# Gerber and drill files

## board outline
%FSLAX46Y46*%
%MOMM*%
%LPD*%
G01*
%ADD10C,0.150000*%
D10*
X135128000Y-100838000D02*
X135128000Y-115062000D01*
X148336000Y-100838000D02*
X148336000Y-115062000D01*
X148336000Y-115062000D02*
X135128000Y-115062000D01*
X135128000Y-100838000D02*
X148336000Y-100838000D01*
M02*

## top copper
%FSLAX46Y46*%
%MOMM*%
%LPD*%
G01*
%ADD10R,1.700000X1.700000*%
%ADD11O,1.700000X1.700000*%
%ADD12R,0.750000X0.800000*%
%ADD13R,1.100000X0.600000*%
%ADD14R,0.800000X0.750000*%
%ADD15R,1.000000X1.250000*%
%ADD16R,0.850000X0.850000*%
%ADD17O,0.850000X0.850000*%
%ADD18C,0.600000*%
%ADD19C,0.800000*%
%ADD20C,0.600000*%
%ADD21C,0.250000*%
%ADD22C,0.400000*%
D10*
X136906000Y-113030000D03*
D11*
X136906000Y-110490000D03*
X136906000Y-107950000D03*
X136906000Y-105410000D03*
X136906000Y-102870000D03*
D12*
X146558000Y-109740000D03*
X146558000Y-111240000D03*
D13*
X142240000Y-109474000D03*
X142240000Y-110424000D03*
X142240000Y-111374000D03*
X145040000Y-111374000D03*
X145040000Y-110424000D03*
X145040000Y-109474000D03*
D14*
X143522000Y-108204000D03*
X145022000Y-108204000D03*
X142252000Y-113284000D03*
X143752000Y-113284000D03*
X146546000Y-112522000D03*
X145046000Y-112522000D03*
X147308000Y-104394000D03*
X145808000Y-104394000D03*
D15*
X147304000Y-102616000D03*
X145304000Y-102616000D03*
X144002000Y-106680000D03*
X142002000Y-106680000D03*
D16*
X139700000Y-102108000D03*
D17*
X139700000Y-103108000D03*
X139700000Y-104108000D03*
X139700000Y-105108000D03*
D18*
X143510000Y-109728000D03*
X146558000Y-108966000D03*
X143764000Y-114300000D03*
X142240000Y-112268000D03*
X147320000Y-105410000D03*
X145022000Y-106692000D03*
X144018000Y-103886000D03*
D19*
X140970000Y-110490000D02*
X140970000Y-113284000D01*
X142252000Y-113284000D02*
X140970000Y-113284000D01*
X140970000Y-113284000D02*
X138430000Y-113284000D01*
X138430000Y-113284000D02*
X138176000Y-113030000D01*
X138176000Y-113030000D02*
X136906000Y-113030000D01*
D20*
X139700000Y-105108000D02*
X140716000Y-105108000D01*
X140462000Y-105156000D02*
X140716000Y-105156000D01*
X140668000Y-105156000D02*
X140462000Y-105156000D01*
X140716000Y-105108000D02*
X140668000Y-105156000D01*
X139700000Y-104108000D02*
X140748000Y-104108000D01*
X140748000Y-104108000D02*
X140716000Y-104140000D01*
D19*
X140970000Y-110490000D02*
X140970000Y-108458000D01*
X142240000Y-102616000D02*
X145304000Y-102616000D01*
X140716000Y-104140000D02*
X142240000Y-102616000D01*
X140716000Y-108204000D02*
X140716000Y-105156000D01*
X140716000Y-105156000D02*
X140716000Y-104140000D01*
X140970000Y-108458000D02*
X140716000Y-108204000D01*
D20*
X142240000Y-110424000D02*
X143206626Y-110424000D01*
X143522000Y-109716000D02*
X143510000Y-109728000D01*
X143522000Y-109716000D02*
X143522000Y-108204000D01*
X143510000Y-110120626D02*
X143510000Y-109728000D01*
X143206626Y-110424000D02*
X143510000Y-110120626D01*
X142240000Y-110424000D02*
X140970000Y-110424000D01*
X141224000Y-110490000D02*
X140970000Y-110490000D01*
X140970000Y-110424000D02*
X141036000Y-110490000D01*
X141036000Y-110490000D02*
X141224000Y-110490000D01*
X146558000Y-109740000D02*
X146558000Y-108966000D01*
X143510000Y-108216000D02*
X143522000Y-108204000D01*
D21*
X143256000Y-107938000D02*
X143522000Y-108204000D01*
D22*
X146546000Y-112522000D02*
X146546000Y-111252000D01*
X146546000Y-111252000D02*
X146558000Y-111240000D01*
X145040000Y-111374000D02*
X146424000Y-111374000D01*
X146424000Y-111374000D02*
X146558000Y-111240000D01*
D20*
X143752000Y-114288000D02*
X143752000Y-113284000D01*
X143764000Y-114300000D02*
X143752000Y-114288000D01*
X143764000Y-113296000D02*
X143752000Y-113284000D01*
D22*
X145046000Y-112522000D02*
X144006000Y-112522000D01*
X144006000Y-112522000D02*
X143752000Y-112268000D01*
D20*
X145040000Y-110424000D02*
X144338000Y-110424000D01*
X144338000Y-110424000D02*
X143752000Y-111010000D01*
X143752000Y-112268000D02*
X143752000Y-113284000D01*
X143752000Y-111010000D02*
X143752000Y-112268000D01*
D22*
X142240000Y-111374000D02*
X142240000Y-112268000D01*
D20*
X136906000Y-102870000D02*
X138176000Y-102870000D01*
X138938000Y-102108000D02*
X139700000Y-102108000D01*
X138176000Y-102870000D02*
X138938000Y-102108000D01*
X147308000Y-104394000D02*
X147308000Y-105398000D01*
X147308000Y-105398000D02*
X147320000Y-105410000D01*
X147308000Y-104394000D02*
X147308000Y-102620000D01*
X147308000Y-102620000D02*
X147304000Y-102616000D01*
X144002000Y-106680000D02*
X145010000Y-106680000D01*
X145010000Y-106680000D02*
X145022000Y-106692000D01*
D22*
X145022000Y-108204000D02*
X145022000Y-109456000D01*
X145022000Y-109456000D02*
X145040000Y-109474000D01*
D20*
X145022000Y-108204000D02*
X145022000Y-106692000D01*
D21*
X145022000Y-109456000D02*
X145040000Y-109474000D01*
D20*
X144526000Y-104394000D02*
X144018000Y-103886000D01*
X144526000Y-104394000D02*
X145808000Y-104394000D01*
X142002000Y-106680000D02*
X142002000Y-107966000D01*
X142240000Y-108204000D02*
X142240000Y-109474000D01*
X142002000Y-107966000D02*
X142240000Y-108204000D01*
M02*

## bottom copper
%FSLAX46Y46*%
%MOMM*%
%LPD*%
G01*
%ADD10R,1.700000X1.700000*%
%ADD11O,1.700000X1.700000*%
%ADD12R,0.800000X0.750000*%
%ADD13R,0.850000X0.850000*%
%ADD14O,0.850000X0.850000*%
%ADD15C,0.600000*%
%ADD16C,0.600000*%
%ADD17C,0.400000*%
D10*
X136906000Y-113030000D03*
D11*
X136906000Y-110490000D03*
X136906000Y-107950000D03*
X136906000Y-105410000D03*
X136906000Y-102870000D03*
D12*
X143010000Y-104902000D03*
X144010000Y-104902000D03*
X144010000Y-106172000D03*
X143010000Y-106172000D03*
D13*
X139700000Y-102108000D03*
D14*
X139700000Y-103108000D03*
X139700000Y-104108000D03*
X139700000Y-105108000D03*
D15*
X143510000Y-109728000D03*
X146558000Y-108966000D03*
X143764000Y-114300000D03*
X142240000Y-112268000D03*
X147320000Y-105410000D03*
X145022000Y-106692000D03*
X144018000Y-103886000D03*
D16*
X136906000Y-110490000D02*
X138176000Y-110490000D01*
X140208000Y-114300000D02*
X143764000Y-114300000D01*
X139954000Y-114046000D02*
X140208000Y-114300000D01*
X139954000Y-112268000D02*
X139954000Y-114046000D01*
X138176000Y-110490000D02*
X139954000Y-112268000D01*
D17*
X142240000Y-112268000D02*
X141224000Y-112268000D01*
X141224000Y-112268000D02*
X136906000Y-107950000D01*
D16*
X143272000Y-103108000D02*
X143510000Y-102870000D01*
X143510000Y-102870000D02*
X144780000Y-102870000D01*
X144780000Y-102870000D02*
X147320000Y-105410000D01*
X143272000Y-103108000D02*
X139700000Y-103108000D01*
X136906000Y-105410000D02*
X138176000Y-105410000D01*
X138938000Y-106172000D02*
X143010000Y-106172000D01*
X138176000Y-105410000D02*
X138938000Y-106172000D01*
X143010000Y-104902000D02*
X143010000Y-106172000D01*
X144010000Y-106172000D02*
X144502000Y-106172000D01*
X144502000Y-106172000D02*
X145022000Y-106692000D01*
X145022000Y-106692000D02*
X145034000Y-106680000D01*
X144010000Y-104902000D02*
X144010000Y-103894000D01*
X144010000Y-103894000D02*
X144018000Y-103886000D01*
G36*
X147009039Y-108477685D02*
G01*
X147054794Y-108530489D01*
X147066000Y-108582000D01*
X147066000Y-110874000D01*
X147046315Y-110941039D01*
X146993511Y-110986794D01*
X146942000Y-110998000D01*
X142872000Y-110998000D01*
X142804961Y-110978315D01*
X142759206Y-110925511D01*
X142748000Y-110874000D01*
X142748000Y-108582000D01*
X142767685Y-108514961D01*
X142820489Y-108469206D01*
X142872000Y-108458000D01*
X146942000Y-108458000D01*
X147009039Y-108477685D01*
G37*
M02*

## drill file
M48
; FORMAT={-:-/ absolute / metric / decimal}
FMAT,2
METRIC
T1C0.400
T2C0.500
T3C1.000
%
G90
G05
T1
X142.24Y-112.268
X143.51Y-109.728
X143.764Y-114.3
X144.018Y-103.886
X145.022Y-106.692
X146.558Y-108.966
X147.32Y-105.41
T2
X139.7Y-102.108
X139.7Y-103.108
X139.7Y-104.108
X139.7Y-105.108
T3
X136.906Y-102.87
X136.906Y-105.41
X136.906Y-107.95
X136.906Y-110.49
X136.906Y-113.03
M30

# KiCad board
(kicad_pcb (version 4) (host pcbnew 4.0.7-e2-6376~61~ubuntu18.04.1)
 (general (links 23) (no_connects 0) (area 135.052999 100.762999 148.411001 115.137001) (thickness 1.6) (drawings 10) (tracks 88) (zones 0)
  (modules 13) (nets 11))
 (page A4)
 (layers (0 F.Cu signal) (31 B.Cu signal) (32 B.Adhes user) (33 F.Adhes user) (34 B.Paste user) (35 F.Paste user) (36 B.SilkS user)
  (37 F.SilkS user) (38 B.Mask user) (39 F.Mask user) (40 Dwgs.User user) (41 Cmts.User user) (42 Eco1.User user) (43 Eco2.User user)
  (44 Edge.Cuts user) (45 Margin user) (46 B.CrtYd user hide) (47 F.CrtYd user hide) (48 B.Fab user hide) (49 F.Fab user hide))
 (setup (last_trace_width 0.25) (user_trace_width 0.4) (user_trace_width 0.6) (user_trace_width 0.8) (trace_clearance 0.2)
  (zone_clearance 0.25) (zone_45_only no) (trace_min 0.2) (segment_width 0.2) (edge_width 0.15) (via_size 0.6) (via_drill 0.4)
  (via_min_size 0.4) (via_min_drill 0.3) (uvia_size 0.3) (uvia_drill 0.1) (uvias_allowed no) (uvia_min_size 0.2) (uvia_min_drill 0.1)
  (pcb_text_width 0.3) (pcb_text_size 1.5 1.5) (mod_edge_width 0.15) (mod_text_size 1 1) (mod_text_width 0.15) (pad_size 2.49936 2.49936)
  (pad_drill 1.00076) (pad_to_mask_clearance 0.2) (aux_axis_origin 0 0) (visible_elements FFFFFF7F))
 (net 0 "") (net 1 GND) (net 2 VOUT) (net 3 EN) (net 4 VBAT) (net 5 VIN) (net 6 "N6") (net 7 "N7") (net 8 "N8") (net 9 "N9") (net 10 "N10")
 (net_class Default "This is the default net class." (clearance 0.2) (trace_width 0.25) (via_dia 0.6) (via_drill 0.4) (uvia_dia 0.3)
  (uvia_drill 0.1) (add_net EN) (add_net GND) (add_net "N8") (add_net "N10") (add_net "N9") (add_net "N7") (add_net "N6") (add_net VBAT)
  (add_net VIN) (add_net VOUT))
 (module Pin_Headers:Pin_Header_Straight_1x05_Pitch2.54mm (layer F.Cu) (at 136.906 113.03 180)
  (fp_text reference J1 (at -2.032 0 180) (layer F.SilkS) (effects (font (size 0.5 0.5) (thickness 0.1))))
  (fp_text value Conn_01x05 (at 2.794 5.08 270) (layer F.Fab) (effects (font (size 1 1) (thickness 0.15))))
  (pad 1 thru_hole rect (at 0 0 180) (size 1.7 1.7) (drill 1) (layers *.Cu *.Mask) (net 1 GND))
  (pad 2 thru_hole oval (at 0 2.54 180) (size 1.7 1.7) (drill 1) (layers *.Cu *.Mask) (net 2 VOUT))
  (pad 3 thru_hole oval (at 0 5.08 180) (size 1.7 1.7) (drill 1) (layers *.Cu *.Mask) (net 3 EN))
  (pad 4 thru_hole oval (at 0 7.62 180) (size 1.7 1.7) (drill 1) (layers *.Cu *.Mask) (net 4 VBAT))
  (pad 5 thru_hole oval (at 0 10.16 180) (size 1.7 1.7) (drill 1) (layers *.Cu *.Mask) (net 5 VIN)))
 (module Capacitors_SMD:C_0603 (layer F.Cu) (at 146.558 110.49 90)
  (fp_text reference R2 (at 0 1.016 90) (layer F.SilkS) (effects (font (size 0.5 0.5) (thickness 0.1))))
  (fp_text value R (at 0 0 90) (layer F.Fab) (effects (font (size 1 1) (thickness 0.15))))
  (pad 2 smd rect (at 0.75 0 90) (size 0.8 0.75) (layers F.Cu F.Paste F.Mask) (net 1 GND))
  (pad 1 smd rect (at -0.75 0 90) (size 0.8 0.75) (layers F.Cu F.Paste F.Mask) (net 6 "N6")))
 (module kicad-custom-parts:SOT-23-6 (layer F.Cu) (at 142.24 109.474 270)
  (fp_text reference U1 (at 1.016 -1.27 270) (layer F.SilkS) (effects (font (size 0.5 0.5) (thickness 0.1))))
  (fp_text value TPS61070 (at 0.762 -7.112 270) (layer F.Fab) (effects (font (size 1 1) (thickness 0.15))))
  (pad 1 smd rect (at 0 0 270) (size 0.6 1.1) (layers F.Cu F.Paste F.Mask) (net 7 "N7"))
  (pad 2 smd rect (at 0.95 0 270) (size 0.6 1.1) (layers F.Cu F.Paste F.Mask) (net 1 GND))
  (pad 3 smd rect (at 1.9 0 270) (size 0.6 1.1) (layers F.Cu F.Paste F.Mask) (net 3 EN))
  (pad 4 smd rect (at 1.9 -2.8 270) (size 0.6 1.1) (layers F.Cu F.Paste F.Mask) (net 6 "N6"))
  (pad 5 smd rect (at 0.95 -2.8 270) (size 0.6 1.1) (layers F.Cu F.Paste F.Mask) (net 2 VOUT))
  (pad 6 smd rect (at 0 -2.8 270) (size 0.6 1.1) (layers F.Cu F.Paste F.Mask) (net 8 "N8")))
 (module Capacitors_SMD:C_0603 (layer F.Cu) (at 144.272 108.204 180)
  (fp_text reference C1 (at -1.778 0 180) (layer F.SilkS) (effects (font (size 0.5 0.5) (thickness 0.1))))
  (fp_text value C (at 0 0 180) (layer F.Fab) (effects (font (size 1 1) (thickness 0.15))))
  (pad 2 smd rect (at 0.75 0 180) (size 0.8 0.75) (layers F.Cu F.Paste F.Mask) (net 1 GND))
  (pad 1 smd rect (at -0.75 0 180) (size 0.8 0.75) (layers F.Cu F.Paste F.Mask) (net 8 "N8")))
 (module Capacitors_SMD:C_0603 (layer F.Cu) (at 143.002 113.284 180)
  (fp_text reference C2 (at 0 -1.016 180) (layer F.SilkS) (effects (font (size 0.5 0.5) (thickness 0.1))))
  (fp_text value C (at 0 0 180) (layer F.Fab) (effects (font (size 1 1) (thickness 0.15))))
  (pad 2 smd rect (at 0.75 0 180) (size 0.8 0.75) (layers F.Cu F.Paste F.Mask) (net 1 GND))
  (pad 1 smd rect (at -0.75 0 180) (size 0.8 0.75) (layers F.Cu F.Paste F.Mask) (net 2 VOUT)))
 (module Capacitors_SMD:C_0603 (layer F.Cu) (at 145.796 112.522)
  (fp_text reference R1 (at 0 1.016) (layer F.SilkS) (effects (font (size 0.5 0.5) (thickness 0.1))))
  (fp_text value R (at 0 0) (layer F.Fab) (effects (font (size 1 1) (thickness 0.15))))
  (pad 2 smd rect (at 0.75 0) (size 0.8 0.75) (layers F.Cu F.Paste F.Mask) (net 6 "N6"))
  (pad 1 smd rect (at -0.75 0) (size 0.8 0.75) (layers F.Cu F.Paste F.Mask) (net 2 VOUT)))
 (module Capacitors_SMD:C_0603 (layer F.Cu) (at 146.558 104.394)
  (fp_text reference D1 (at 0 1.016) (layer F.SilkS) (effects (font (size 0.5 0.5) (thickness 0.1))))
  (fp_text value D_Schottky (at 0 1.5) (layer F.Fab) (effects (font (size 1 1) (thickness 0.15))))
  (pad 2 smd rect (at 0.75 0) (size 0.8 0.75) (layers F.Cu F.Paste F.Mask) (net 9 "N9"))
  (pad 1 smd rect (at -0.75 0) (size 0.8 0.75) (layers F.Cu F.Paste F.Mask) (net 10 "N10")))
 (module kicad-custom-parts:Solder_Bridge (layer B.Cu) (at 143.51 104.902 180)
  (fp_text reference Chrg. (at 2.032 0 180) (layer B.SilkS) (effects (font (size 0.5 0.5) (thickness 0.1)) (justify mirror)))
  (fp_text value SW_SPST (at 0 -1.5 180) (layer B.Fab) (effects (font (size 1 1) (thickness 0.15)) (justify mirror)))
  (pad 2 smd rect (at 0.5 0 180) (size 0.8 0.75) (layers B.Cu B.Paste B.Mask) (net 4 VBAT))
  (pad 1 smd rect (at -0.5 0 180) (size 0.8 0.75) (layers B.Cu B.Paste B.Mask) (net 10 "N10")))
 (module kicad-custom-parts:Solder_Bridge (layer B.Cu) (at 143.51 106.172)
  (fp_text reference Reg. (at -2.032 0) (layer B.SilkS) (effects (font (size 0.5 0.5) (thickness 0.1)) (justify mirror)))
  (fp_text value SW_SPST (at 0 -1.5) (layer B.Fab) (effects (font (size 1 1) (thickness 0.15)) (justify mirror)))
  (pad 2 smd rect (at 0.5 0) (size 0.8 0.75) (layers B.Cu B.Paste B.Mask) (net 8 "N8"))
  (pad 1 smd rect (at -0.5 0) (size 0.8 0.75) (layers B.Cu B.Paste B.Mask) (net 4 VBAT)))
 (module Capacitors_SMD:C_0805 (layer F.Cu) (at 146.304 102.616 180)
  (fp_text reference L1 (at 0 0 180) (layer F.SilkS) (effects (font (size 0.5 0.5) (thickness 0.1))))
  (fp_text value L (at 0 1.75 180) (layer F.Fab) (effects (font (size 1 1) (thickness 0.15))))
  (pad 1 smd rect (at -1 0 180) (size 1 1.25) (layers F.Cu F.Paste F.Mask) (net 9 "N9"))
  (pad 2 smd rect (at 1 0 180) (size 1 1.25) (layers F.Cu F.Paste F.Mask) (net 1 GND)))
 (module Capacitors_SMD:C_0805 (layer F.Cu) (at 143.002 106.68 180)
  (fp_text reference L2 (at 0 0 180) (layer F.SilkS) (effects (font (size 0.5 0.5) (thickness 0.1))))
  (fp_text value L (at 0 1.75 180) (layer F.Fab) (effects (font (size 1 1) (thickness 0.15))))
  (pad 1 smd rect (at -1 0 180) (size 1 1.25) (layers F.Cu F.Paste F.Mask) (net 8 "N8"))
  (pad 2 smd rect (at 1 0 180) (size 1 1.25) (layers F.Cu F.Paste F.Mask) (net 7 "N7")))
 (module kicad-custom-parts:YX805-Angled (layer F.Cu) (at 139.7 102.108)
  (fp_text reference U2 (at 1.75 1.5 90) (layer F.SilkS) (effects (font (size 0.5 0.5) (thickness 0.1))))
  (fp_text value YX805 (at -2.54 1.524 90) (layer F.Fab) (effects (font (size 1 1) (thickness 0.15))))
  (pad 1 thru_hole rect (at 0 0) (size 0.85 0.85) (drill 0.5) (layers *.Cu *.Mask) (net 5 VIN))
  (pad 2 thru_hole oval (at 0 1) (size 0.85 0.85) (drill 0.5) (layers *.Cu *.Mask) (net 9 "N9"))
  (pad 3 thru_hole oval (at 0 2) (size 0.85 0.85) (drill 0.5) (layers *.Cu *.Mask) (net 1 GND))
  (pad 4 thru_hole oval (at 0 3) (size 0.85 0.85) (drill 0.5) (layers *.Cu *.Mask) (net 1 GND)))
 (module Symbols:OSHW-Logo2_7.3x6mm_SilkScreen (layer B.Cu) (at 142.494 110.998 270)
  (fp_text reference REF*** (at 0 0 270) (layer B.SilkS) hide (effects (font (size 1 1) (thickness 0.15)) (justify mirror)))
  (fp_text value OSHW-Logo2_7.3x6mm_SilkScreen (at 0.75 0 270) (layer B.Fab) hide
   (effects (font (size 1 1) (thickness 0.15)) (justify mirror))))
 (gr_line (start 135.128 100.838) (end 135.128 115.062) (angle 90) (layer Edge.Cuts) (width 0.15))
 (gr_line (start 148.336 100.838) (end 148.336 115.062) (angle 90) (layer Edge.Cuts) (width 0.15))
 (gr_line (start 148.336 115.062) (end 135.128 115.062) (angle 90) (layer Edge.Cuts) (width 0.15))
 (gr_line (start 135.128 100.838) (end 148.336 100.838) (angle 90) (layer Edge.Cuts) (width 0.15))
 (segment (start 140.97 110.49) (end 140.97 113.284) (width 0.8) (layer F.Cu) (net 1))
 (segment (start 142.252 113.284) (end 140.97 113.284) (width 0.8) (layer F.Cu) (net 1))
 (segment (start 140.97 113.284) (end 138.43 113.284) (width 0.8) (layer F.Cu) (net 1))
 (segment (start 138.43 113.284) (end 138.176 113.03) (width 0.8) (layer F.Cu) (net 1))
 (segment (start 138.176 113.03) (end 136.906 113.03) (width 0.8) (layer F.Cu) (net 1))
 (segment (start 139.7 105.108) (end 140.716 105.108) (width 0.6) (layer F.Cu) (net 1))
 (segment (start 140.462 105.156) (end 140.716 105.156) (width 0.6) (layer F.Cu) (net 1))
 (segment (start 140.668 105.156) (end 140.462 105.156) (width 0.6) (layer F.Cu) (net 1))
 (segment (start 140.716 105.108) (end 140.668 105.156) (width 0.6) (layer F.Cu) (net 1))
 (segment (start 139.7 104.108) (end 140.748 104.108) (width 0.6) (layer F.Cu) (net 1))
 (segment (start 140.748 104.108) (end 140.716 104.14) (width 0.6) (layer F.Cu) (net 1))
 (segment (start 140.97 110.49) (end 140.97 108.458) (width 0.8) (layer F.Cu) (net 1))
 (segment (start 142.24 102.616) (end 145.304 102.616) (width 0.8) (layer F.Cu) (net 1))
 (segment (start 140.716 104.14) (end 142.24 102.616) (width 0.8) (layer F.Cu) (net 1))
 (segment (start 140.716 108.204) (end 140.716 105.156) (width 0.8) (layer F.Cu) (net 1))
 (segment (start 140.716 105.156) (end 140.716 104.14) (width 0.8) (layer F.Cu) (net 1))
 (segment (start 140.97 108.458) (end 140.716 108.204) (width 0.8) (layer F.Cu) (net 1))
 (segment (start 142.24 110.424) (end 143.206626 110.424) (width 0.6) (layer F.Cu) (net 1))
 (segment (start 143.522 109.716) (end 143.51 109.728) (width 0.6) (layer F.Cu) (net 1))
 (via (at 143.51 109.728) (size 0.6) (drill 0.4) (layers F.Cu B.Cu) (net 1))
 (segment (start 143.522 109.716) (end 143.522 108.204) (width 0.6) (layer F.Cu) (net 1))
 (segment (start 143.51 110.120626) (end 143.51 109.728) (width 0.6) (layer F.Cu) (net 1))
 (segment (start 143.206626 110.424) (end 143.51 110.120626) (width 0.6) (layer F.Cu) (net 1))
 (segment (start 142.24 110.424) (end 140.97 110.424) (width 0.6) (layer F.Cu) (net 1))
 (segment (start 141.224 110.49) (end 140.97 110.49) (width 0.6) (layer F.Cu) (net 1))
 (segment (start 140.97 110.424) (end 141.036 110.49) (width 0.6) (layer F.Cu) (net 1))
 (segment (start 141.036 110.49) (end 141.224 110.49) (width 0.6) (layer F.Cu) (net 1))
 (segment (start 146.558 109.74) (end 146.558 108.966) (width 0.6) (layer F.Cu) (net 1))
 (via (at 146.558 108.966) (size 0.6) (drill 0.4) (layers F.Cu B.Cu) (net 1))
 (segment (start 143.51 108.216) (end 143.522 108.204) (width 0.6) (layer F.Cu) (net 1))
 (segment (start 143.256 107.938) (end 143.522 108.204) (width 0.25) (layer F.Cu) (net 1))
 (segment (start 146.546 112.522) (end 146.546 111.252) (width 0.4) (layer F.Cu) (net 6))
 (segment (start 146.546 111.252) (end 146.558 111.24) (width 0.4) (layer F.Cu) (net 6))
 (segment (start 145.04 111.374) (end 146.424 111.374) (width 0.4) (layer F.Cu) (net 6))
 (segment (start 146.424 111.374) (end 146.558 111.24) (width 0.4) (layer F.Cu) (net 6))
 (segment (start 136.906 110.49) (end 138.176 110.49) (width 0.6) (layer B.Cu) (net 2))
 (segment (start 143.752 114.288) (end 143.752 113.284) (width 0.6) (layer F.Cu) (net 2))
 (segment (start 143.764 114.3) (end 143.752 114.288) (width 0.6) (layer F.Cu) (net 2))
 (via (at 143.764 114.3) (size 0.6) (drill 0.4) (layers F.Cu B.Cu) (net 2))
 (segment (start 140.208 114.3) (end 143.764 114.3) (width 0.6) (layer B.Cu) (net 2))
 (segment (start 139.954 114.046) (end 140.208 114.3) (width 0.6) (layer B.Cu) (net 2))
 (segment (start 139.954 112.268) (end 139.954 114.046) (width 0.6) (layer B.Cu) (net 2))
 (segment (start 138.176 110.49) (end 139.954 112.268) (width 0.6) (layer B.Cu) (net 2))
 (segment (start 143.764 113.296) (end 143.752 113.284) (width 0.6) (layer F.Cu) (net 2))
 (segment (start 145.046 112.522) (end 144.006 112.522) (width 0.4) (layer F.Cu) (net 2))
 (segment (start 144.006 112.522) (end 143.752 112.268) (width 0.4) (layer F.Cu) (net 2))
 (segment (start 145.04 110.424) (end 144.338 110.424) (width 0.6) (layer F.Cu) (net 2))
 (segment (start 144.338 110.424) (end 143.752 111.01) (width 0.6) (layer F.Cu) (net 2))
 (segment (start 143.752 112.268) (end 143.752 113.284) (width 0.6) (layer F.Cu) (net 2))
 (segment (start 143.752 111.01) (end 143.752 112.268) (width 0.6) (layer F.Cu) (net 2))
 (segment (start 142.24 112.268) (end 141.224 112.268) (width 0.4) (layer B.Cu) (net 3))
 (via (at 142.24 112.268) (size 0.6) (drill 0.4) (layers F.Cu B.Cu) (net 3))
 (segment (start 142.24 111.374) (end 142.24 112.268) (width 0.4) (layer F.Cu) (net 3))
 (segment (start 141.224 112.268) (end 136.906 107.95) (width 0.4) (layer B.Cu) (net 3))
 (segment (start 136.906 102.87) (end 138.176 102.87) (width 0.6) (layer F.Cu) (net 5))
 (segment (start 138.938 102.108) (end 139.7 102.108) (width 0.6) (layer F.Cu) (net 5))
 (segment (start 138.176 102.87) (end 138.938 102.108) (width 0.6) (layer F.Cu) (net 5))
 (segment (start 147.308 104.394) (end 147.308 105.398) (width 0.6) (layer F.Cu) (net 9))
 (segment (start 143.272 103.108) (end 143.51 102.87) (width 0.6) (layer B.Cu) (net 9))
 (segment (start 143.51 102.87) (end 144.78 102.87) (width 0.6) (layer B.Cu) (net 9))
 (segment (start 144.78 102.87) (end 147.32 105.41) (width 0.6) (layer B.Cu) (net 9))
 (via (at 147.32 105.41) (size 0.6) (drill 0.4) (layers F.Cu B.Cu) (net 9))
 (segment (start 143.272 103.108) (end 139.7 103.108) (width 0.6) (layer B.Cu) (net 9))
 (segment (start 147.308 105.398) (end 147.32 105.41) (width 0.6) (layer F.Cu) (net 9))
 (segment (start 147.308 104.394) (end 147.308 102.62) (width 0.6) (layer F.Cu) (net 9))
 (segment (start 147.308 102.62) (end 147.304 102.616) (width 0.6) (layer F.Cu) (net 9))
 (segment (start 136.906 105.41) (end 138.176 105.41) (width 0.6) (layer B.Cu) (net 4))
 (segment (start 138.938 106.172) (end 143.01 106.172) (width 0.6) (layer B.Cu) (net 4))
 (segment (start 138.176 105.41) (end 138.938 106.172) (width 0.6) (layer B.Cu) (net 4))
 (segment (start 143.01 104.902) (end 143.01 106.172) (width 0.6) (layer B.Cu) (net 4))
 (segment (start 144.002 106.68) (end 145.01 106.68) (width 0.6) (layer F.Cu) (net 8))
 (segment (start 145.01 106.68) (end 145.022 106.692) (width 0.6) (layer F.Cu) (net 8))
 (segment (start 145.022 108.204) (end 145.022 109.456) (width 0.4) (layer F.Cu) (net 8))
 (segment (start 145.022 109.456) (end 145.04 109.474) (width 0.4) (layer F.Cu) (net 8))
 (segment (start 144.01 106.172) (end 144.502 106.172) (width 0.6) (layer B.Cu) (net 8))
 (segment (start 144.502 106.172) (end 145.022 106.692) (width 0.6) (layer B.Cu) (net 8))
 (segment (start 145.022 108.204) (end 145.022 106.692) (width 0.6) (layer F.Cu) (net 8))
 (segment (start 145.022 109.456) (end 145.04 109.474) (width 0.25) (layer F.Cu) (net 8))
 (via (at 145.022 106.692) (size 0.6) (drill 0.4) (layers F.Cu B.Cu) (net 8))
 (segment (start 145.022 106.692) (end 145.034 106.68) (width 0.6) (layer B.Cu) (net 8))
 (segment (start 144.01 104.902) (end 144.01 103.894) (width 0.6) (layer B.Cu) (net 10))
 (segment (start 144.526 104.394) (end 144.018 103.886) (width 0.6) (layer F.Cu) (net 10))
 (via (at 144.018 103.886) (size 0.6) (drill 0.4) (layers F.Cu B.Cu) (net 10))
 (segment (start 144.526 104.394) (end 145.808 104.394) (width 0.6) (layer F.Cu) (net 10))
 (segment (start 144.01 103.894) (end 144.018 103.886) (width 0.6) (layer B.Cu) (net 10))
 (segment (start 142.002 106.68) (end 142.002 107.966) (width 0.6) (layer F.Cu) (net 7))
 (segment (start 142.24 108.204) (end 142.24 109.474) (width 0.6) (layer F.Cu) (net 7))
 (segment (start 142.002 107.966) (end 142.24 108.204) (width 0.6) (layer F.Cu) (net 7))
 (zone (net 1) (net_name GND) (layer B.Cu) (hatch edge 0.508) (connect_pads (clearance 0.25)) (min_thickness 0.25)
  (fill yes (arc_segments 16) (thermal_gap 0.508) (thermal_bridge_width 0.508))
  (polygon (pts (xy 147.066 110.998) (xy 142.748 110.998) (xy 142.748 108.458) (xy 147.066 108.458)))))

